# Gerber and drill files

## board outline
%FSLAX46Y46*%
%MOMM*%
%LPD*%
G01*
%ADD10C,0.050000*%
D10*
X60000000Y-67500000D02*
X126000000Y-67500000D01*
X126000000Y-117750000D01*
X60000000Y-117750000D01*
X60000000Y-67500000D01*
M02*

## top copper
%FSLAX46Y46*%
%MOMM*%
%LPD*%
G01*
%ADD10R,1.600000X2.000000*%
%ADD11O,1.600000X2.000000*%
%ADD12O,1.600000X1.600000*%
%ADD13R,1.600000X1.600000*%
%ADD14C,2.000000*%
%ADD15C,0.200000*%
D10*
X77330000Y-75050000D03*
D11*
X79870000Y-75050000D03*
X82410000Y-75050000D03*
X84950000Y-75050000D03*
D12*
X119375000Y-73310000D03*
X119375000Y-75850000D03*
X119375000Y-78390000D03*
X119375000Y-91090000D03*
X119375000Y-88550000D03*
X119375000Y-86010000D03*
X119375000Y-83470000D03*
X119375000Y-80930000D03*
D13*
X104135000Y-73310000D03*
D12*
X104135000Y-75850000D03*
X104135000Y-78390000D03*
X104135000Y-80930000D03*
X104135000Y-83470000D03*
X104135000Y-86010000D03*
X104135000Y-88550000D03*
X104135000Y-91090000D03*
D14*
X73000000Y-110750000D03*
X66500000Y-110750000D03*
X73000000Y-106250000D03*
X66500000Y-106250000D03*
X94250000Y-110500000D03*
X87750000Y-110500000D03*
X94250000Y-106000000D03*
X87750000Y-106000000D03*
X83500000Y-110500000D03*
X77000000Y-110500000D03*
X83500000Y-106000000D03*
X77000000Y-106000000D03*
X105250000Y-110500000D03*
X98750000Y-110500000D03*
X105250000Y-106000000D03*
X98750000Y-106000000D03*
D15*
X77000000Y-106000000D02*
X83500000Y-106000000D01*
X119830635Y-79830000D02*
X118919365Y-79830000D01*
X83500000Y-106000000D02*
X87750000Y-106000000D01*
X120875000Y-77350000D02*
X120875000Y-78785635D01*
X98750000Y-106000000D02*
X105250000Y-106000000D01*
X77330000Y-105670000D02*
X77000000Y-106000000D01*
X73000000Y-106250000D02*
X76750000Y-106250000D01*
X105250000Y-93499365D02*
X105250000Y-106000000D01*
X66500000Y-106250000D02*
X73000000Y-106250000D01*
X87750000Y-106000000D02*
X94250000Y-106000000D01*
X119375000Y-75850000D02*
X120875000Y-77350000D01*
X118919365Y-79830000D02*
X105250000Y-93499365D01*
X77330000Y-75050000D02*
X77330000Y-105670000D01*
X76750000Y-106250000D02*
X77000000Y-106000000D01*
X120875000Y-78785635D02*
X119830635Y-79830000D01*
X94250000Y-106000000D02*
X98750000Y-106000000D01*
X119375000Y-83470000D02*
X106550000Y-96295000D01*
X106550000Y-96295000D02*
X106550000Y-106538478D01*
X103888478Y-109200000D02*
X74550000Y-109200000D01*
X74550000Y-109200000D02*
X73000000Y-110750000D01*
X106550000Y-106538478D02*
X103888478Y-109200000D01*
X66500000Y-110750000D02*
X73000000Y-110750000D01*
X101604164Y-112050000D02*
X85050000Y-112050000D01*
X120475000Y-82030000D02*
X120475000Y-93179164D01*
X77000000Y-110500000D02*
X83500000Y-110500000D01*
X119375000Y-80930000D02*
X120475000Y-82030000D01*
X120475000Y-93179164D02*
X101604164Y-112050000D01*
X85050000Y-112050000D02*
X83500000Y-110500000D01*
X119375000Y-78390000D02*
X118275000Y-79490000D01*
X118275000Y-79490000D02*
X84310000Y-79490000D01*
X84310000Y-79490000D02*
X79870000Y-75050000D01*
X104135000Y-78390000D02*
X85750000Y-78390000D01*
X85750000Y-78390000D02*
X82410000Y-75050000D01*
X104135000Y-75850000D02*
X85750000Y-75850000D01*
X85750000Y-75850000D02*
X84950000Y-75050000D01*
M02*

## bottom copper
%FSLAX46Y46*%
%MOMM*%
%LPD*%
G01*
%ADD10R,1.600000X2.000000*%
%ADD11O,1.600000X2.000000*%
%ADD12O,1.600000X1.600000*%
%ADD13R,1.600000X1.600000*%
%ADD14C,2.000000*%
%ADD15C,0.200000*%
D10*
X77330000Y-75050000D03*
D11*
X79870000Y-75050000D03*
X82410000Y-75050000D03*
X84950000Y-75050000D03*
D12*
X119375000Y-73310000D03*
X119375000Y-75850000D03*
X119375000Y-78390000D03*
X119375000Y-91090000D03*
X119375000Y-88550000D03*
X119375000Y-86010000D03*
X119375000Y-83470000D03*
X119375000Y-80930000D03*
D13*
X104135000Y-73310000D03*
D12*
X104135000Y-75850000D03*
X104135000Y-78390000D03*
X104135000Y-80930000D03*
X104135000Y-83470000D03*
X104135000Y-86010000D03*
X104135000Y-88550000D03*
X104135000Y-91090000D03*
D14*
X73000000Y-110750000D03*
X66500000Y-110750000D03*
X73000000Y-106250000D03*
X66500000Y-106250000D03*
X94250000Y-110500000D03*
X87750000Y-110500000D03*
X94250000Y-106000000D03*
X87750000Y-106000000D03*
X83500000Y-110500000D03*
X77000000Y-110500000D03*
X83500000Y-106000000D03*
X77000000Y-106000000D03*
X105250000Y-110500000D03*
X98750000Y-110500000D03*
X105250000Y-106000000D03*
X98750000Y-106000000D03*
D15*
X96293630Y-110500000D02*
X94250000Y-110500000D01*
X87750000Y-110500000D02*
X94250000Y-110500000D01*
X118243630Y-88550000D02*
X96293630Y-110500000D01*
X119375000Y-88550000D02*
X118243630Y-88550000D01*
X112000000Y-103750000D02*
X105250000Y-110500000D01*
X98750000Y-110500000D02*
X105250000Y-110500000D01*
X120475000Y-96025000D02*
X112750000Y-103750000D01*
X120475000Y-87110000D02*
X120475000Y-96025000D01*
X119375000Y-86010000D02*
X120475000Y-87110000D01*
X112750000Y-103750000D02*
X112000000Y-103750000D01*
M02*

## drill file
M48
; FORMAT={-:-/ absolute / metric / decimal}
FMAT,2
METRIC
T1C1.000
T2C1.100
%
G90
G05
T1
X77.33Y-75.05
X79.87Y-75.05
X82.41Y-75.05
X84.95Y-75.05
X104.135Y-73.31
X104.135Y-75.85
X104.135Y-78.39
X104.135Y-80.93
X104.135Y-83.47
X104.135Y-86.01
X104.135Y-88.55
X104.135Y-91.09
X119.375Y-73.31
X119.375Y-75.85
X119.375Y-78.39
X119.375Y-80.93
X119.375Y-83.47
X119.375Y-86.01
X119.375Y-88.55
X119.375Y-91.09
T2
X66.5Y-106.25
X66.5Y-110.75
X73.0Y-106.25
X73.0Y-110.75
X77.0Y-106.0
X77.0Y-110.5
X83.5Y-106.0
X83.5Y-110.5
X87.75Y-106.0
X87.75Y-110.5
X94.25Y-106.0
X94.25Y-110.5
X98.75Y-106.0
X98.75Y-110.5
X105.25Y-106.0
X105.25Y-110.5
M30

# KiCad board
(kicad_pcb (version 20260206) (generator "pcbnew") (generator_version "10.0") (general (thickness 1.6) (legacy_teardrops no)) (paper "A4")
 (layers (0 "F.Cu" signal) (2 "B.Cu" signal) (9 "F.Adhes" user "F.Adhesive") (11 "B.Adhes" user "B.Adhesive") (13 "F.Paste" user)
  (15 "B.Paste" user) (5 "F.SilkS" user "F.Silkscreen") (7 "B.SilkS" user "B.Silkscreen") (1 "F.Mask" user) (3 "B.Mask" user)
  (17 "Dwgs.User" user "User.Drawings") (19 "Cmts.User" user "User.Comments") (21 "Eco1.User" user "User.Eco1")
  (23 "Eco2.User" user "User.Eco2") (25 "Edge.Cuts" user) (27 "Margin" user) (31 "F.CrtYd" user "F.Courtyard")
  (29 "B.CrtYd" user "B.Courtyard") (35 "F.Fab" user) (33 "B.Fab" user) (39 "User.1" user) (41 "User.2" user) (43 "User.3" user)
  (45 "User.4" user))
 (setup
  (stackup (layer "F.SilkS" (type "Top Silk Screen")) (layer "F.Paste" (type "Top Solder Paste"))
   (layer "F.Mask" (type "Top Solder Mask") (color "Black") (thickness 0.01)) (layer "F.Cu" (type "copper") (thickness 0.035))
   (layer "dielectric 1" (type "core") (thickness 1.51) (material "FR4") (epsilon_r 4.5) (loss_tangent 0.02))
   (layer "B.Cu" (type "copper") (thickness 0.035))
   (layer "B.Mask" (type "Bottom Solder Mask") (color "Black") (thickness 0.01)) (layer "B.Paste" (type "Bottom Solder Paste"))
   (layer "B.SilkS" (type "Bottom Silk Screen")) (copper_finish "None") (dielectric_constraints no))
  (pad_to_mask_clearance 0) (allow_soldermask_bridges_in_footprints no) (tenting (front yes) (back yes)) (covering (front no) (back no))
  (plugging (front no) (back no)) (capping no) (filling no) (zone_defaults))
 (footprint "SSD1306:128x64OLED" (layer "F.Cu") (at 80.95 85.65)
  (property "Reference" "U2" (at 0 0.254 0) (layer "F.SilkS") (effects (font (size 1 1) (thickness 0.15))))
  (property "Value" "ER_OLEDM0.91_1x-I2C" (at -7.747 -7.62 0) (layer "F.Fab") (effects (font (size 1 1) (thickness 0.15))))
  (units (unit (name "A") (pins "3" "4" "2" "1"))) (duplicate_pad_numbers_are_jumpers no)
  (pad "1" thru_hole rect (at -3.62 -10.6 90) (size 2 1.6) (drill 1) (layers "*.Cu" "*.Mask") (remove_unused_layers no) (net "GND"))
  (pad "2" thru_hole oval (at -1.08 -10.6 90) (size 2 1.6) (drill 1) (layers "*.Cu" "*.Mask") (remove_unused_layers no)
   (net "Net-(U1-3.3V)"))
  (pad "3" thru_hole oval (at 1.46 -10.6 90) (size 2 1.6) (drill 1) (layers "*.Cu" "*.Mask") (remove_unused_layers no) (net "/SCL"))
  (pad "4" thru_hole oval (at 4 -10.6 90) (size 2 1.6) (drill 1) (layers "*.Cu" "*.Mask") (remove_unused_layers no) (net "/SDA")))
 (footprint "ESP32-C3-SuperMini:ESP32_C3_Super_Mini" (layer "F.Cu") (at 104.135 73.31)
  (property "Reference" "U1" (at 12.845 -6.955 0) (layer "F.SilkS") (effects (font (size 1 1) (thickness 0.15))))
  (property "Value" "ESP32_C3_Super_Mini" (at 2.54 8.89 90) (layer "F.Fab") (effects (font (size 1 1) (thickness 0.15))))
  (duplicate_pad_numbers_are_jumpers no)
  (pad "-1" thru_hole oval (at 15.24 0) (size 1.6 1.6) (drill 1) (layers "*.Cu" "*.Mask") (remove_unused_layers no) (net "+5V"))
  (pad "-2" thru_hole oval (at 15.24 2.54) (size 1.6 1.6) (drill 1) (layers "*.Cu" "*.Mask") (remove_unused_layers no) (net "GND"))
  (pad "-3" thru_hole oval (at 15.24 5.08) (size 1.6 1.6) (drill 1) (layers "*.Cu" "*.Mask") (remove_unused_layers no) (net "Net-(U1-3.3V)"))
  (pad "0" thru_hole oval (at 15.24 17.78) (size 1.6 1.6) (drill 1) (layers "*.Cu" "*.Mask") (remove_unused_layers no)
   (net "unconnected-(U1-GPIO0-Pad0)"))
  (pad "1" thru_hole oval (at 15.24 15.24) (size 1.6 1.6) (drill 1) (layers "*.Cu" "*.Mask") (remove_unused_layers no) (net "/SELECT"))
  (pad "2" thru_hole oval (at 15.24 12.7) (size 1.6 1.6) (drill 1) (layers "*.Cu" "*.Mask") (remove_unused_layers no) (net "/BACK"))
  (pad "3" thru_hole oval (at 15.24 10.16) (size 1.6 1.6) (drill 1) (layers "*.Cu" "*.Mask") (remove_unused_layers no) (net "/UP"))
  (pad "4" thru_hole oval (at 15.24 7.62) (size 1.6 1.6) (drill 1) (layers "*.Cu" "*.Mask") (remove_unused_layers no) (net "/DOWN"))
  (pad "5" thru_hole rect (at 0 0) (size 1.6 1.6) (drill 1) (layers "*.Cu" "*.Mask") (remove_unused_layers no)
   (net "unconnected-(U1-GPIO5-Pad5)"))
  (pad "6" thru_hole oval (at 0 2.54) (size 1.6 1.6) (drill 1) (layers "*.Cu" "*.Mask") (remove_unused_layers no) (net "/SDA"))
  (pad "7" thru_hole oval (at 0 5.08) (size 1.6 1.6) (drill 1) (layers "*.Cu" "*.Mask") (remove_unused_layers no) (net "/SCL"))
  (pad "8" thru_hole oval (at 0 7.62) (size 1.6 1.6) (drill 1) (layers "*.Cu" "*.Mask") (remove_unused_layers no)
   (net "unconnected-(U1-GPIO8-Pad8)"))
  (pad "9" thru_hole oval (at 0 10.16) (size 1.6 1.6) (drill 1) (layers "*.Cu" "*.Mask") (remove_unused_layers no)
   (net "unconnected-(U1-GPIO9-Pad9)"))
  (pad "10" thru_hole oval (at 0 12.7) (size 1.6 1.6) (drill 1) (layers "*.Cu" "*.Mask") (remove_unused_layers no)
   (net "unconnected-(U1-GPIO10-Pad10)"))
  (pad "20" thru_hole oval (at 0 15.24) (size 1.6 1.6) (drill 1) (layers "*.Cu" "*.Mask") (remove_unused_layers no)
   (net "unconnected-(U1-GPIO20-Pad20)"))
  (pad "21" thru_hole oval (at 0 17.78) (size 1.6 1.6) (drill 1) (layers "*.Cu" "*.Mask") (remove_unused_layers no)
   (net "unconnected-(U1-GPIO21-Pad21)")))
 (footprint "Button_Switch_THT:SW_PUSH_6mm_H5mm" (layer "F.Cu") (at 73 110.75 180)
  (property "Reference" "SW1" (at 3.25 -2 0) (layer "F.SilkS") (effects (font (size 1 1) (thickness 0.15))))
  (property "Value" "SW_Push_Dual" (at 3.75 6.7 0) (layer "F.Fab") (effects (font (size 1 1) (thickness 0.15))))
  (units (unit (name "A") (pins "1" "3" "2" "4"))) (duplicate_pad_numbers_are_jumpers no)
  (pad "1" thru_hole circle (at 0 0 270) (size 2 2) (drill 1.1) (layers "*.Cu" "*.Mask") (remove_unused_layers no) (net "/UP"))
  (pad "1" thru_hole circle (at 6.5 0 270) (size 2 2) (drill 1.1) (layers "*.Cu" "*.Mask") (remove_unused_layers no) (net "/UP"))
  (pad "2" thru_hole circle (at 0 4.5 270) (size 2 2) (drill 1.1) (layers "*.Cu" "*.Mask") (remove_unused_layers no) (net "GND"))
  (pad "2" thru_hole circle (at 6.5 4.5 270) (size 2 2) (drill 1.1) (layers "*.Cu" "*.Mask") (remove_unused_layers no) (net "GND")))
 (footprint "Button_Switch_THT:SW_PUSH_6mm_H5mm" (layer "F.Cu") (at 94.25 110.5 180)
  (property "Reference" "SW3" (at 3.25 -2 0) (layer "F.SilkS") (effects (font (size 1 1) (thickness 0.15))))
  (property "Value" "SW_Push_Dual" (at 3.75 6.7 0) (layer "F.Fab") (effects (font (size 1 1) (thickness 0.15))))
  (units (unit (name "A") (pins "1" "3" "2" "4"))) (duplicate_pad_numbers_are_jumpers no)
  (pad "1" thru_hole circle (at 0 0 270) (size 2 2) (drill 1.1) (layers "*.Cu" "*.Mask") (remove_unused_layers no) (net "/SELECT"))
  (pad "1" thru_hole circle (at 6.5 0 270) (size 2 2) (drill 1.1) (layers "*.Cu" "*.Mask") (remove_unused_layers no) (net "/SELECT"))
  (pad "2" thru_hole circle (at 0 4.5 270) (size 2 2) (drill 1.1) (layers "*.Cu" "*.Mask") (remove_unused_layers no) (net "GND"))
  (pad "2" thru_hole circle (at 6.5 4.5 270) (size 2 2) (drill 1.1) (layers "*.Cu" "*.Mask") (remove_unused_layers no) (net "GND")))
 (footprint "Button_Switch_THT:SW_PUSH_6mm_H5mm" (layer "F.Cu") (at 83.5 110.5 180)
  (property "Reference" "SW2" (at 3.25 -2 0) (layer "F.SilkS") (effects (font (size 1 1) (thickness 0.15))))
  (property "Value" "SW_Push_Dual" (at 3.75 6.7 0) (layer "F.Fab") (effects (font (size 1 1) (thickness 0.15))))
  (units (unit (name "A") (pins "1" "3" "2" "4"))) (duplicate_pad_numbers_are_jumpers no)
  (pad "1" thru_hole circle (at 0 0 270) (size 2 2) (drill 1.1) (layers "*.Cu" "*.Mask") (remove_unused_layers no) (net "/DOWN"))
  (pad "1" thru_hole circle (at 6.5 0 270) (size 2 2) (drill 1.1) (layers "*.Cu" "*.Mask") (remove_unused_layers no) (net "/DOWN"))
  (pad "2" thru_hole circle (at 0 4.5 270) (size 2 2) (drill 1.1) (layers "*.Cu" "*.Mask") (remove_unused_layers no) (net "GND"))
  (pad "2" thru_hole circle (at 6.5 4.5 270) (size 2 2) (drill 1.1) (layers "*.Cu" "*.Mask") (remove_unused_layers no) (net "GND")))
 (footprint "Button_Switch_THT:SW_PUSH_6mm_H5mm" (layer "F.Cu") (at 105.25 110.5 180)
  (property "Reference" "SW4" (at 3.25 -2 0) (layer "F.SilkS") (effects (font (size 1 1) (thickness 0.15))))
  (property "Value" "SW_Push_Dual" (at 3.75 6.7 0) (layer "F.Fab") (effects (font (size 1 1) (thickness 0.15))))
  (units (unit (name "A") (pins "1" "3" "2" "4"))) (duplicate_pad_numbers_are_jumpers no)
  (pad "1" thru_hole circle (at 0 0 270) (size 2 2) (drill 1.1) (layers "*.Cu" "*.Mask") (remove_unused_layers no) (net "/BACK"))
  (pad "1" thru_hole circle (at 6.5 0 270) (size 2 2) (drill 1.1) (layers "*.Cu" "*.Mask") (remove_unused_layers no) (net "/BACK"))
  (pad "2" thru_hole circle (at 0 4.5 270) (size 2 2) (drill 1.1) (layers "*.Cu" "*.Mask") (remove_unused_layers no) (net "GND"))
  (pad "2" thru_hole circle (at 6.5 4.5 270) (size 2 2) (drill 1.1) (layers "*.Cu" "*.Mask") (remove_unused_layers no) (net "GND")))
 (gr_rect (start 60 67.5) (end 126 117.75) (stroke (width 0.05) (type default)) (fill no) (layer "Edge.Cuts"))
 (segment (start 77 106) (end 83.5 106) (width 0.2) (layer "F.Cu") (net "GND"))
 (segment (start 119.830635 79.83) (end 118.919365 79.83) (width 0.2) (layer "F.Cu") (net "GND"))
 (segment (start 83.5 106) (end 87.75 106) (width 0.2) (layer "F.Cu") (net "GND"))
 (segment (start 120.875 77.35) (end 120.875 78.785635) (width 0.2) (layer "F.Cu") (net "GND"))
 (segment (start 98.75 106) (end 105.25 106) (width 0.2) (layer "F.Cu") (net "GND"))
 (segment (start 77.33 105.67) (end 77 106) (width 0.2) (layer "F.Cu") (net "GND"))
 (segment (start 73 106.25) (end 76.75 106.25) (width 0.2) (layer "F.Cu") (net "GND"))
 (segment (start 105.25 93.499365) (end 105.25 106) (width 0.2) (layer "F.Cu") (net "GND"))
 (segment (start 66.5 106.25) (end 73 106.25) (width 0.2) (layer "F.Cu") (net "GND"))
 (segment (start 87.75 106) (end 94.25 106) (width 0.2) (layer "F.Cu") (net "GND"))
 (segment (start 119.375 75.85) (end 120.875 77.35) (width 0.2) (layer "F.Cu") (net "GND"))
 (segment (start 118.919365 79.83) (end 105.25 93.499365) (width 0.2) (layer "F.Cu") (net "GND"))
 (segment (start 77.33 75.05) (end 77.33 105.67) (width 0.2) (layer "F.Cu") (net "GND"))
 (segment (start 76.75 106.25) (end 77 106) (width 0.2) (layer "F.Cu") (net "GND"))
 (segment (start 120.875 78.785635) (end 119.830635 79.83) (width 0.2) (layer "F.Cu") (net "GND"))
 (segment (start 94.25 106) (end 98.75 106) (width 0.2) (layer "F.Cu") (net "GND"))
 (segment (start 119.375 83.47) (end 106.55 96.295) (width 0.2) (layer "F.Cu") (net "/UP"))
 (segment (start 106.55 96.295) (end 106.55 106.538478) (width 0.2) (layer "F.Cu") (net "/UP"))
 (segment (start 103.888478 109.2) (end 74.55 109.2) (width 0.2) (layer "F.Cu") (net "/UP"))
 (segment (start 74.55 109.2) (end 73 110.75) (width 0.2) (layer "F.Cu") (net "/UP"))
 (segment (start 106.55 106.538478) (end 103.888478 109.2) (width 0.2) (layer "F.Cu") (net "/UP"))
 (segment (start 66.5 110.75) (end 73 110.75) (width 0.2) (layer "F.Cu") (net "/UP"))
 (segment (start 101.604164 112.05) (end 85.05 112.05) (width 0.2) (layer "F.Cu") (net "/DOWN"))
 (segment (start 120.475 82.03) (end 120.475 93.179164) (width 0.2) (layer "F.Cu") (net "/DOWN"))
 (segment (start 77 110.5) (end 83.5 110.5) (width 0.2) (layer "F.Cu") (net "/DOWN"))
 (segment (start 119.375 80.93) (end 120.475 82.03) (width 0.2) (layer "F.Cu") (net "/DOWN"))
 (segment (start 120.475 93.179164) (end 101.604164 112.05) (width 0.2) (layer "F.Cu") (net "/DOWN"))
 (segment (start 85.05 112.05) (end 83.5 110.5) (width 0.2) (layer "F.Cu") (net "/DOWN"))
 (segment (start 96.29363 110.5) (end 94.25 110.5) (width 0.2) (layer "B.Cu") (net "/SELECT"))
 (segment (start 87.75 110.5) (end 94.25 110.5) (width 0.2) (layer "B.Cu") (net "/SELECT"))
 (segment (start 118.24363 88.55) (end 96.29363 110.5) (width 0.2) (layer "B.Cu") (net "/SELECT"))
 (segment (start 119.375 88.55) (end 118.24363 88.55) (width 0.2) (layer "B.Cu") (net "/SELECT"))
 (segment (start 112 103.75) (end 105.25 110.5) (width 0.2) (layer "B.Cu") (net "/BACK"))
 (segment (start 98.75 110.5) (end 105.25 110.5) (width 0.2) (layer "B.Cu") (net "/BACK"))
 (segment (start 120.475 96.025) (end 112.75 103.75) (width 0.2) (layer "B.Cu") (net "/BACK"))
 (segment (start 120.475 87.11) (end 120.475 96.025) (width 0.2) (layer "B.Cu") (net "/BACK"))
 (segment (start 119.375 86.01) (end 120.475 87.11) (width 0.2) (layer "B.Cu") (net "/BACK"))
 (segment (start 112.75 103.75) (end 112 103.75) (width 0.2) (layer "B.Cu") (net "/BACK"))
 (segment (start 119.375 78.39) (end 118.275 79.49) (width 0.2) (layer "F.Cu") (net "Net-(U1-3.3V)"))
 (segment (start 118.275 79.49) (end 84.31 79.49) (width 0.2) (layer "F.Cu") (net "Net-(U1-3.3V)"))
 (segment (start 84.31 79.49) (end 79.87 75.05) (width 0.2) (layer "F.Cu") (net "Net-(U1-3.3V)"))
 (segment (start 104.135 78.39) (end 85.75 78.39) (width 0.2) (layer "F.Cu") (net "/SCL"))
 (segment (start 85.75 78.39) (end 82.41 75.05) (width 0.2) (layer "F.Cu") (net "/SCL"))
 (segment (start 104.135 75.85) (end 85.75 75.85) (width 0.2) (layer "F.Cu") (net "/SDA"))
 (segment (start 85.75 75.85) (end 84.95 75.05) (width 0.2) (layer "F.Cu") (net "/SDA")))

